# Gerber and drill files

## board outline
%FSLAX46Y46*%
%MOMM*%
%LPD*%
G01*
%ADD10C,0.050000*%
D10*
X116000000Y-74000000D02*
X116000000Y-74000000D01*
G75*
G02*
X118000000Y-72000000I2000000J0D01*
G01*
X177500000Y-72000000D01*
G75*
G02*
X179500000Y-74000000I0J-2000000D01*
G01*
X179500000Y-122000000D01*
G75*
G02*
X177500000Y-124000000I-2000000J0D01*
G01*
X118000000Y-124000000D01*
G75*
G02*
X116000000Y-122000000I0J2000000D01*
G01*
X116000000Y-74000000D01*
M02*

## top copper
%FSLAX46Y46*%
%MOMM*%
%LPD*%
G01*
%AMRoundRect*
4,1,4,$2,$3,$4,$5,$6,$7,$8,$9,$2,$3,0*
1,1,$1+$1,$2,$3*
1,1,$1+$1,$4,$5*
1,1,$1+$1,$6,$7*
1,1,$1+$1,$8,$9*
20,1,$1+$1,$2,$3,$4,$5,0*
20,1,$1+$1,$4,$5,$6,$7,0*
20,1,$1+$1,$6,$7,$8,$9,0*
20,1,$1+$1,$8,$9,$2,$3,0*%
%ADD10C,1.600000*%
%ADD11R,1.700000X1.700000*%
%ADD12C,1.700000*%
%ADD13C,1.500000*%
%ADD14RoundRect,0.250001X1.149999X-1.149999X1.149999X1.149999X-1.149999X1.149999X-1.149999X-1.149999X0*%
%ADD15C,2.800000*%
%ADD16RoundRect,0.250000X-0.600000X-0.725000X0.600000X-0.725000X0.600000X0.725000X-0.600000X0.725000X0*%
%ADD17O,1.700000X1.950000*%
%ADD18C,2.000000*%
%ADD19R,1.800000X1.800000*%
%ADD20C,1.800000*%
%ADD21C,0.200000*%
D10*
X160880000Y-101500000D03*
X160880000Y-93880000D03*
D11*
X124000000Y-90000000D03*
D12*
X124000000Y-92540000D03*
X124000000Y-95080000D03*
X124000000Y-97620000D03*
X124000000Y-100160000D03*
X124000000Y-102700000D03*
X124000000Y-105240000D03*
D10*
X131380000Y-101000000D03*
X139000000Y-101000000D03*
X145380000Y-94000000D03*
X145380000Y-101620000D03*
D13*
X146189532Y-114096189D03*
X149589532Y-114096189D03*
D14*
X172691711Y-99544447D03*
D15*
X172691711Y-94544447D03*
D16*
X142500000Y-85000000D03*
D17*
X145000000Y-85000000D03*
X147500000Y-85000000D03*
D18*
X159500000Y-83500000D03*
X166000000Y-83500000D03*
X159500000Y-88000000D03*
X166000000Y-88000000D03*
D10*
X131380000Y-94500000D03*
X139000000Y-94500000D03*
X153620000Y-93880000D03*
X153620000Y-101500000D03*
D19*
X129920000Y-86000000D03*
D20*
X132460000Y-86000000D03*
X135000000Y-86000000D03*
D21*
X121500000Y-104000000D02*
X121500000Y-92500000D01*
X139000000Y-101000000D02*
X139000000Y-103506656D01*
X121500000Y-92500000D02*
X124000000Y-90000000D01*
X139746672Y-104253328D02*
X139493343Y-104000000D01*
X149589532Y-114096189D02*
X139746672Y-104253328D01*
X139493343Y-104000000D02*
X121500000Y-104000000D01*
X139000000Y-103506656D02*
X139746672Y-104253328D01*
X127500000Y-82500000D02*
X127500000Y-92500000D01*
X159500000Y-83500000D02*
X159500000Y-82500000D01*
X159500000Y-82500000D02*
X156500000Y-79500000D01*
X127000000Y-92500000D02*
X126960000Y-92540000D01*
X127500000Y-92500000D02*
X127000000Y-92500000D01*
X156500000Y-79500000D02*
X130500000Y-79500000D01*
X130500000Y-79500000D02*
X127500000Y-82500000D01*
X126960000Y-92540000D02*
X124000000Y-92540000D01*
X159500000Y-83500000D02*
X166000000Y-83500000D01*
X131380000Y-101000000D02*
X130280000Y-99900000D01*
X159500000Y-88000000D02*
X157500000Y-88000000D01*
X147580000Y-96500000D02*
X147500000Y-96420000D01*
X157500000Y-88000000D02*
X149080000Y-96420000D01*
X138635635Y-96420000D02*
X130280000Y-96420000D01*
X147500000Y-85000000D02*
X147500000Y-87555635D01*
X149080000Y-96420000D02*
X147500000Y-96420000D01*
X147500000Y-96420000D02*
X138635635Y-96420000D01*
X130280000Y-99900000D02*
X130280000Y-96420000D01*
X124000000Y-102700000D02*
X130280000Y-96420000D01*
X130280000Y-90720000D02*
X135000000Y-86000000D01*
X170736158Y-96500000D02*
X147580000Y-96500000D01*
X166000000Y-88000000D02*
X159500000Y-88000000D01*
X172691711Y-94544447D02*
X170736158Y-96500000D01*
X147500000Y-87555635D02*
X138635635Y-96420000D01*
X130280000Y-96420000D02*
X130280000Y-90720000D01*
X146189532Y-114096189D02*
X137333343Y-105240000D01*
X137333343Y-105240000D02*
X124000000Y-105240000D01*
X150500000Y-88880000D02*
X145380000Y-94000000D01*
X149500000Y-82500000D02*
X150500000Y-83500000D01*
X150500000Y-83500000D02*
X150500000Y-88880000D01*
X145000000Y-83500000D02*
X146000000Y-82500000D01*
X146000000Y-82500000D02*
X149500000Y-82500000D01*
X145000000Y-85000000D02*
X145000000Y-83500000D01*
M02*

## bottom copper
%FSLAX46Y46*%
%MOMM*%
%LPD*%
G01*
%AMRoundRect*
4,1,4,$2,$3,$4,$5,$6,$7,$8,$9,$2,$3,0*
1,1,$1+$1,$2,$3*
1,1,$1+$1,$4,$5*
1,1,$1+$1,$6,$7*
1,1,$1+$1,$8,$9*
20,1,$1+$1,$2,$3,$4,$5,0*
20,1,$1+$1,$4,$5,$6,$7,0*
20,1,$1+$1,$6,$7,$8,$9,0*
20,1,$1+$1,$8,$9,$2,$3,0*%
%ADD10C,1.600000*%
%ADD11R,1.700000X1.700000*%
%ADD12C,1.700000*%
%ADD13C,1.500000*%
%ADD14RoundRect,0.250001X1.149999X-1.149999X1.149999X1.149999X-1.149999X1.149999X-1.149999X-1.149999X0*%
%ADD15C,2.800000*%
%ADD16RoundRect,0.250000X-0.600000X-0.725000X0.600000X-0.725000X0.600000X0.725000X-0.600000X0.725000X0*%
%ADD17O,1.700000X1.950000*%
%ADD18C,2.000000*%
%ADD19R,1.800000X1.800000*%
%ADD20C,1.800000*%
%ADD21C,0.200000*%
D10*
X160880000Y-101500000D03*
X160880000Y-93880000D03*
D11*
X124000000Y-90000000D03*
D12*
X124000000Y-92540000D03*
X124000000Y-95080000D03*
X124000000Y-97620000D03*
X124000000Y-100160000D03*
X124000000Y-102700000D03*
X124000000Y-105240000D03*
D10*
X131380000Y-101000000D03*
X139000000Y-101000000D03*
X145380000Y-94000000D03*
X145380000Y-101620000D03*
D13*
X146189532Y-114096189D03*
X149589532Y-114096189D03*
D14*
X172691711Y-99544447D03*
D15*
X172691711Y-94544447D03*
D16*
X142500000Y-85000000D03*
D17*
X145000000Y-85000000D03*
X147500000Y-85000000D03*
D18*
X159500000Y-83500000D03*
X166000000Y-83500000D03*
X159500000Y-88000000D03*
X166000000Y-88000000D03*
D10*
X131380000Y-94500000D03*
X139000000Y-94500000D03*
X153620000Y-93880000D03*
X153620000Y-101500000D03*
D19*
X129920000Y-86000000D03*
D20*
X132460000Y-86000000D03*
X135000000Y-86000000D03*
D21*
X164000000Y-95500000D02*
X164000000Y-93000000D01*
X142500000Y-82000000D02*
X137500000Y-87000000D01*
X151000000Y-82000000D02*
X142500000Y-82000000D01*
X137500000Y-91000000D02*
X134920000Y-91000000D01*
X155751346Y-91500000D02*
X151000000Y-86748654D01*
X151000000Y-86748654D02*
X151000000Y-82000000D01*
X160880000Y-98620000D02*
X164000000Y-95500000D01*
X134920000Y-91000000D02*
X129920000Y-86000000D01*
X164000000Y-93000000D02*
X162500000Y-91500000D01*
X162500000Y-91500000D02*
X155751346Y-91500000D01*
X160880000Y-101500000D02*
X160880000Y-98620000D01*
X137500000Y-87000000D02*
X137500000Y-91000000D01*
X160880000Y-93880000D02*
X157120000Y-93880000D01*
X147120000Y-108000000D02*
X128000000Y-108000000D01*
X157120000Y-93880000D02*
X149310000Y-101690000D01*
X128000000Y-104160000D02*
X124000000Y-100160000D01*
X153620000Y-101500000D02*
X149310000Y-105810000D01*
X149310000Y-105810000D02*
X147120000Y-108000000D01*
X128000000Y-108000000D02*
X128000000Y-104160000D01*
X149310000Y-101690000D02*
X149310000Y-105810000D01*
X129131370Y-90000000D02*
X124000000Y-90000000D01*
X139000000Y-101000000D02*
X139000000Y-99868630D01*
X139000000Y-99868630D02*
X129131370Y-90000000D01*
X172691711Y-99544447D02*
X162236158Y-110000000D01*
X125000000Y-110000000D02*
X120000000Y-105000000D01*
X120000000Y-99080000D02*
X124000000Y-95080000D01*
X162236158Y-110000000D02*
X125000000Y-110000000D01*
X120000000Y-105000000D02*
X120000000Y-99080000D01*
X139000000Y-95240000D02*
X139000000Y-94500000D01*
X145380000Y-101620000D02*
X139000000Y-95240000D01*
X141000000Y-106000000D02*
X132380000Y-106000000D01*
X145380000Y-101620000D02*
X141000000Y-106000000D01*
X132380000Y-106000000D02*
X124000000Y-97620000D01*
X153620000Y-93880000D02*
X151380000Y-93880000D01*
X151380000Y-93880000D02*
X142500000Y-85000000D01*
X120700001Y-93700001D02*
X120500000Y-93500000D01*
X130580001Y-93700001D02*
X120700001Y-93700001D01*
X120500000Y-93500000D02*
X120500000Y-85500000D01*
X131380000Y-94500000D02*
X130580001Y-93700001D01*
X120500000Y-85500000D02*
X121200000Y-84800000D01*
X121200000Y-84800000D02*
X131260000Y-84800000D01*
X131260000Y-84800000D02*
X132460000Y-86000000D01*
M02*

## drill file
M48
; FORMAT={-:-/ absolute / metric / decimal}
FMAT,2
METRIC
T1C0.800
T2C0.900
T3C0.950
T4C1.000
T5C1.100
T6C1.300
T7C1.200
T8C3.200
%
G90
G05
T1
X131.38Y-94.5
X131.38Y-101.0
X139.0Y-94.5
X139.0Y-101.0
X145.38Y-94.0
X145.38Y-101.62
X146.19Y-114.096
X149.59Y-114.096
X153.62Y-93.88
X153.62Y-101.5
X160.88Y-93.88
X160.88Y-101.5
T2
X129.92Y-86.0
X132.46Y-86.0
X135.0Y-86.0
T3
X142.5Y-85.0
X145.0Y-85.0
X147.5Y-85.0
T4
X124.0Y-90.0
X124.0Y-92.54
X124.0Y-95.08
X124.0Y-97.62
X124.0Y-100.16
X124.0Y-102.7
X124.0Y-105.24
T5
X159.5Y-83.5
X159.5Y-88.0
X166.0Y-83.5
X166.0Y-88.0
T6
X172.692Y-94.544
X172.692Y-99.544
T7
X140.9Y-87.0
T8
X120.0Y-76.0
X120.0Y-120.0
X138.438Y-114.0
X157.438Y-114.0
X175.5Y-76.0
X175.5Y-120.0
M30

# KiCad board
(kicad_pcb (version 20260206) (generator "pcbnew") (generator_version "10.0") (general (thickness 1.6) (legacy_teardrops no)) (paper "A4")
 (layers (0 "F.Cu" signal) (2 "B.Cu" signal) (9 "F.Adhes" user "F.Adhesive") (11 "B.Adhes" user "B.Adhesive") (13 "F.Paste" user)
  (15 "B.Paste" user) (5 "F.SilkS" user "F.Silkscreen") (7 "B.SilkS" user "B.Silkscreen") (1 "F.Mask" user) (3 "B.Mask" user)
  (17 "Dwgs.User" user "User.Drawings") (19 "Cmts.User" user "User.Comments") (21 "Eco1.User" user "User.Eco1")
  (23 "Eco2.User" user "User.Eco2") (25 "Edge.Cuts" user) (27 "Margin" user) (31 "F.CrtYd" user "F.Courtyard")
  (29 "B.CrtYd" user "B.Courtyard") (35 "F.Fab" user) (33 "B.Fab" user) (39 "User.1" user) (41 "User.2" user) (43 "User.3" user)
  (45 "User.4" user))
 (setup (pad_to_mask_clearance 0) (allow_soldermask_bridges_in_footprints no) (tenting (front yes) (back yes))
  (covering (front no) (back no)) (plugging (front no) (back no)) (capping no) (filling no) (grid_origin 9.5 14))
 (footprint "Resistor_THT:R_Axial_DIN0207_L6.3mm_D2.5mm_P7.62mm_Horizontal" (layer "F.Cu") (at 160.88 101.5 90)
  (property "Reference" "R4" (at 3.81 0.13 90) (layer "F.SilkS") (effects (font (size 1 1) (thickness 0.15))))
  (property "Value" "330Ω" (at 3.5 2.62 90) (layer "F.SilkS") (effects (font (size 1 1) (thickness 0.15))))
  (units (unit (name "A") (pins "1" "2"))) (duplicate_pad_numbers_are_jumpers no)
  (pad "1" thru_hole circle (at 0 0 90) (size 1.6 1.6) (drill 0.8) (layers "*.Cu" "*.Mask") (remove_unused_layers no) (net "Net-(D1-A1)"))
  (pad "2" thru_hole circle (at 7.62 0 90) (size 1.6 1.6) (drill 0.8) (layers "*.Cu" "*.Mask") (remove_unused_layers no) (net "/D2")))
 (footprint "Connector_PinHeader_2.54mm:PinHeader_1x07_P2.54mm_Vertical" (layer "F.Cu") (at 124 90)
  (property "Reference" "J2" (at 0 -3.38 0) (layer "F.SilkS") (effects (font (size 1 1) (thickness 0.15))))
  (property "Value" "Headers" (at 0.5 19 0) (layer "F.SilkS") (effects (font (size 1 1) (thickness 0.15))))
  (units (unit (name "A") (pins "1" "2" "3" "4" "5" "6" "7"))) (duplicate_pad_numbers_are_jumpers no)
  (pad "1" thru_hole rect (at 0 0) (size 1.7 1.7) (drill 1) (layers "*.Cu" "*.Mask") (remove_unused_layers no) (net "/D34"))
  (pad "2" thru_hole circle (at 0 2.54) (size 1.7 1.7) (drill 1) (layers "*.Cu" "*.Mask") (remove_unused_layers no) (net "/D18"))
  (pad "3" thru_hole circle (at 0 5.08) (size 1.7 1.7) (drill 1) (layers "*.Cu" "*.Mask") (remove_unused_layers no) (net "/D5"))
  (pad "4" thru_hole circle (at 0 7.62) (size 1.7 1.7) (drill 1) (layers "*.Cu" "*.Mask") (remove_unused_layers no) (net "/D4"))
  (pad "5" thru_hole circle (at 0 10.16) (size 1.7 1.7) (drill 1) (layers "*.Cu" "*.Mask") (remove_unused_layers no) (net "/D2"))
  (pad "6" thru_hole circle (at 0 12.7) (size 1.7 1.7) (drill 1) (layers "*.Cu" "*.Mask") (remove_unused_layers no) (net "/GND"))
  (pad "7" thru_hole circle (at 0 15.24) (size 1.7 1.7) (drill 1) (layers "*.Cu" "*.Mask") (remove_unused_layers no) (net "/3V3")))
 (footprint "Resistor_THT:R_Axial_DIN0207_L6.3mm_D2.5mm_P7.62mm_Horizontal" (layer "F.Cu") (at 131.38 101)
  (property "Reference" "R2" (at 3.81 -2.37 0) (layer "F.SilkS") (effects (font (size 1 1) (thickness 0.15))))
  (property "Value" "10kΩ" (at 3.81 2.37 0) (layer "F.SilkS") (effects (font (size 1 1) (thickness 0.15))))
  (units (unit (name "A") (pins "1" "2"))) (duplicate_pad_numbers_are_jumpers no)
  (pad "1" thru_hole circle (at 0 0) (size 1.6 1.6) (drill 0.8) (layers "*.Cu" "*.Mask") (remove_unused_layers no) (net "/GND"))
  (pad "2" thru_hole circle (at 7.62 0) (size 1.6 1.6) (drill 0.8) (layers "*.Cu" "*.Mask") (remove_unused_layers no) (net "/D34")))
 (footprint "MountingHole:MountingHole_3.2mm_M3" (layer "F.Cu") (at 175.5 120)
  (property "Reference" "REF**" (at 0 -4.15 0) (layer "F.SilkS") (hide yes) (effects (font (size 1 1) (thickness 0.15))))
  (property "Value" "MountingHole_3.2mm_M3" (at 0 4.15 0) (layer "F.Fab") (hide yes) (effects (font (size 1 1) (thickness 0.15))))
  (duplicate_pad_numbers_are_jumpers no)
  (pad "" np_thru_hole circle (at 0 0) (size 3.2 3.2) (drill 3.2) (layers "*.Cu" "*.Mask")))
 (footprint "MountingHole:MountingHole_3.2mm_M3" (layer "F.Cu") (at 175.5 76)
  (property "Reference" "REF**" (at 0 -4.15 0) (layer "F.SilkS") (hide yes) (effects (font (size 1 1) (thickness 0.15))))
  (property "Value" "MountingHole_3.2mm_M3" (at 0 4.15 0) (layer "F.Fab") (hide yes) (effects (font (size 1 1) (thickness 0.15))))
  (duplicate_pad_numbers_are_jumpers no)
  (pad "" np_thru_hole circle (at 0 0) (size 3.2 3.2) (drill 3.2) (layers "*.Cu" "*.Mask")))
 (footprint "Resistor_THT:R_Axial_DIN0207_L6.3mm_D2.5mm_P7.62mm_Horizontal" (layer "F.Cu") (at 145.38 94 -90)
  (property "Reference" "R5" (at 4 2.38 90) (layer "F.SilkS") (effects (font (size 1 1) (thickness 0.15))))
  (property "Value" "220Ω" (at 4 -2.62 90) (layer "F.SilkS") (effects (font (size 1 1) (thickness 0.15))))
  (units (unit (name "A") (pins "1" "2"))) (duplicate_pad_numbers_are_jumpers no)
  (pad "1" thru_hole circle (at 0 0 270) (size 1.6 1.6) (drill 0.8) (layers "*.Cu" "*.Mask") (remove_unused_layers no)
   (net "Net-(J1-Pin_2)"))
  (pad "2" thru_hole circle (at 7.62 0 270) (size 1.6 1.6) (drill 0.8) (layers "*.Cu" "*.Mask") (remove_unused_layers no) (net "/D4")))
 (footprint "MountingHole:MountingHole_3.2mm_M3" (layer "F.Cu") (at 157.437676 114)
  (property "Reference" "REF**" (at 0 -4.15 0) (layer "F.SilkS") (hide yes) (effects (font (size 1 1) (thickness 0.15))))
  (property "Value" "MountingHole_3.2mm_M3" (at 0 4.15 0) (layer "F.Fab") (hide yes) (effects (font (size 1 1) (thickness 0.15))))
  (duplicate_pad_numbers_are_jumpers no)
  (pad "" np_thru_hole circle (at 0 0) (size 3.2 3.2) (drill 3.2) (layers "*.Cu" "*.Mask")))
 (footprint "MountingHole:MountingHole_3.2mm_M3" (layer "F.Cu") (at 120 76)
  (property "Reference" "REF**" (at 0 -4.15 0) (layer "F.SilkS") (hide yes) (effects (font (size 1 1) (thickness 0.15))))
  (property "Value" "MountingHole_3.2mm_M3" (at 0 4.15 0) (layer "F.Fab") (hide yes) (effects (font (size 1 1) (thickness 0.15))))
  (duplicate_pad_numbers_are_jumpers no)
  (pad "" np_thru_hole circle (at 0 0) (size 3.2 3.2) (drill 3.2) (layers "*.Cu" "*.Mask")))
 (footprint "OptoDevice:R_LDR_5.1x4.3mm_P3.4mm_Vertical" (layer "F.Cu") (at 146.189532 114.096189)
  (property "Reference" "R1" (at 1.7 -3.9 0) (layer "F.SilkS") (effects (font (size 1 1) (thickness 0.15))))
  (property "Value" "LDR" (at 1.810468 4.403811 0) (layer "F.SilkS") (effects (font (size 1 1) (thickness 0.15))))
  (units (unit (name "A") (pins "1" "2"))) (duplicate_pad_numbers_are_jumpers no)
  (pad "1" thru_hole circle (at 0 0) (size 1.5 1.5) (drill 0.8) (layers "*.Cu" "*.Mask") (remove_unused_layers no) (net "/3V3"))
  (pad "2" thru_hole circle (at 3.4 0) (size 1.5 1.5) (drill 0.8) (layers "*.Cu" "*.Mask") (remove_unused_layers no) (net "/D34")))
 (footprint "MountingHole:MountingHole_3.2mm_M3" (layer "F.Cu") (at 120 120)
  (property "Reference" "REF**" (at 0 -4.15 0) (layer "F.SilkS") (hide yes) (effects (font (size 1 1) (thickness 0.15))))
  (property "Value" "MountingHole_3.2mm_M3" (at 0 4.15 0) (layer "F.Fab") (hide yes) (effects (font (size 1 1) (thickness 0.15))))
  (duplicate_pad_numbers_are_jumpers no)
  (pad "" np_thru_hole circle (at 0 0) (size 3.2 3.2) (drill 3.2) (layers "*.Cu" "*.Mask")))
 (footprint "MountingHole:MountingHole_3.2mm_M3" (layer "F.Cu") (at 138.437676 114)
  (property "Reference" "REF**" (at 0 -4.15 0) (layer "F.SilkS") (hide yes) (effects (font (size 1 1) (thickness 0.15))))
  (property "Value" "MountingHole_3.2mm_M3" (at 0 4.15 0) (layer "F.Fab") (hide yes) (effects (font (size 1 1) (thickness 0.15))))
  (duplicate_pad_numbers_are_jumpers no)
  (pad "" np_thru_hole circle (at 0 0) (size 3.2 3.2) (drill 3.2) (layers "*.Cu" "*.Mask")))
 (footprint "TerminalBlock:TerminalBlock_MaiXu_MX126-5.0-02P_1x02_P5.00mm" (layer "F.Cu") (at 172.691711 99.544447 90)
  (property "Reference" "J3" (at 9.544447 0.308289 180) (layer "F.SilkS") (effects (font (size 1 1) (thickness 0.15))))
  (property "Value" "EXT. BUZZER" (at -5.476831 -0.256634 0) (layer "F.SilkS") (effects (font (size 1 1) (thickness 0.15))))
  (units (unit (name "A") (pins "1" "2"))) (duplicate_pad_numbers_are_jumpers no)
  (pad "1" thru_hole roundrect (at 0 0 90) (size 2.8 2.8) (drill 1.3) (layers "*.Cu" "*.Mask") (remove_unused_layers no)
   (roundrect_rratio 0.089286) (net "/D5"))
  (pad "2" thru_hole circle (at 5 0 90) (size 2.8 2.8) (drill 1.3) (layers "*.Cu" "*.Mask") (remove_unused_layers no) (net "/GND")))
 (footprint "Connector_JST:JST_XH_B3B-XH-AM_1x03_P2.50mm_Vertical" (layer "F.Cu") (at 142.5 85)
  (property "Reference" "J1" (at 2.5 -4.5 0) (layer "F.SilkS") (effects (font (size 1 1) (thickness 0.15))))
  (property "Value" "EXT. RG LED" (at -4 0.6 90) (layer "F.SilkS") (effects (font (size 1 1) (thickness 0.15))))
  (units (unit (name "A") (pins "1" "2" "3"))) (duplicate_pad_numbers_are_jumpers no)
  (pad "" np_thru_hole circle (at -1.6 2) (size 1.2 1.2) (drill 1.2) (layers "*.Cu" "*.Mask"))
  (pad "1" thru_hole roundrect (at 0 0) (size 1.7 1.95) (drill 0.95) (layers "*.Cu" "*.Mask") (remove_unused_layers no)
   (roundrect_rratio 0.147059) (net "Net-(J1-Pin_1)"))
  (pad "2" thru_hole oval (at 2.5 0) (size 1.7 1.95) (drill 0.95) (layers "*.Cu" "*.Mask") (remove_unused_layers no) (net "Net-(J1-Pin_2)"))
  (pad "3" thru_hole oval (at 5 0) (size 1.7 1.95) (drill 0.95) (layers "*.Cu" "*.Mask") (remove_unused_layers no) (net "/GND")))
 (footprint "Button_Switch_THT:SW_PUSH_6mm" (layer "F.Cu") (at 159.5 83.5)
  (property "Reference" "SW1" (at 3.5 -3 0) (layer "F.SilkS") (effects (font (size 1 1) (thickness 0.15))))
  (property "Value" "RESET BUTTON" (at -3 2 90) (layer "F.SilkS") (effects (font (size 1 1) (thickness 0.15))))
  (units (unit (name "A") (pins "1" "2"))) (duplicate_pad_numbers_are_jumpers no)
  (pad "1" thru_hole circle (at 0 0 90) (size 2 2) (drill 1.1) (layers "*.Cu" "*.Mask") (remove_unused_layers no) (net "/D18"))
  (pad "1" thru_hole circle (at 6.5 0 90) (size 2 2) (drill 1.1) (layers "*.Cu" "*.Mask") (remove_unused_layers no) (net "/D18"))
  (pad "2" thru_hole circle (at 0 4.5 90) (size 2 2) (drill 1.1) (layers "*.Cu" "*.Mask") (remove_unused_layers no) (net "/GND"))
  (pad "2" thru_hole circle (at 6.5 4.5 90) (size 2 2) (drill 1.1) (layers "*.Cu" "*.Mask") (remove_unused_layers no) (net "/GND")))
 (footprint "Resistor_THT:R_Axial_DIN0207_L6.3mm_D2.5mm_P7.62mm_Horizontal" (layer "F.Cu") (at 131.38 94.5)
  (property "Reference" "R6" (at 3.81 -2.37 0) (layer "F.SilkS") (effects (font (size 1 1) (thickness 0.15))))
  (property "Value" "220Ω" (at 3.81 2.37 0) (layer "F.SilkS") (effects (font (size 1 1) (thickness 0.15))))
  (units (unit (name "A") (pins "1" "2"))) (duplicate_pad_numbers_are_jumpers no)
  (pad "1" thru_hole circle (at 0 0) (size 1.6 1.6) (drill 0.8) (layers "*.Cu" "*.Mask") (remove_unused_layers no) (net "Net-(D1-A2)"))
  (pad "2" thru_hole circle (at 7.62 0) (size 1.6 1.6) (drill 0.8) (layers "*.Cu" "*.Mask") (remove_unused_layers no) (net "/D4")))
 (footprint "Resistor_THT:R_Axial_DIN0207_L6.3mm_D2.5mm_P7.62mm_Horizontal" (layer "F.Cu") (at 153.62 93.88 -90)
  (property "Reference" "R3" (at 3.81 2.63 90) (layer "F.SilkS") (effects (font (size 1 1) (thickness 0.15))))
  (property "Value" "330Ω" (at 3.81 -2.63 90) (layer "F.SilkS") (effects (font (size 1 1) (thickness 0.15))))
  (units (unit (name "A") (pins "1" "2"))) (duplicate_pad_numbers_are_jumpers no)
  (pad "1" thru_hole circle (at 0 0 270) (size 1.6 1.6) (drill 0.8) (layers "*.Cu" "*.Mask") (remove_unused_layers no)
   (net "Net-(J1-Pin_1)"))
  (pad "2" thru_hole circle (at 7.62 0 270) (size 1.6 1.6) (drill 0.8) (layers "*.Cu" "*.Mask") (remove_unused_layers no) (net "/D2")))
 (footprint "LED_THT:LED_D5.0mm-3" (layer "F.Cu") (at 129.92 86)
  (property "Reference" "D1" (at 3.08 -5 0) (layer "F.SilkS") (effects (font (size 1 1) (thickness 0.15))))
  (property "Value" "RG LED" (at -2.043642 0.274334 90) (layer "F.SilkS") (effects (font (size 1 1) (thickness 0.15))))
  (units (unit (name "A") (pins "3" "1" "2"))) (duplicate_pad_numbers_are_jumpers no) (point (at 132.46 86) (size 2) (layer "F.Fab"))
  (pad "1" thru_hole rect (at 0 0) (size 1.8 1.8) (drill 0.9) (layers "*.Cu" "*.Mask") (remove_unused_layers no) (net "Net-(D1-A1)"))
  (pad "2" thru_hole circle (at 2.54 0) (size 1.8 1.8) (drill 0.9) (layers "*.Cu" "*.Mask") (remove_unused_layers no) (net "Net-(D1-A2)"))
  (pad "3" thru_hole circle (at 5.08 0) (size 1.8 1.8) (drill 0.9) (layers "*.Cu" "*.Mask") (remove_unused_layers no) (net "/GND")))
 (gr_rect (start 116 72) (end 179.5 124) (radius 2) (stroke (width 0.05) (type default)) (fill no) (layer "Edge.Cuts"))
 (segment (start 164 95.5) (end 164 93) (width 0.2) (layer "B.Cu") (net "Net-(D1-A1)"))
 (segment (start 142.5 82) (end 137.5 87) (width 0.2) (layer "B.Cu") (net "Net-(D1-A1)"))
 (segment (start 151 82) (end 142.5 82) (width 0.2) (layer "B.Cu") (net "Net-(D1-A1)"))
 (segment (start 137.5 91) (end 134.92 91) (width 0.2) (layer "B.Cu") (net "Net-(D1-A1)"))
 (segment (start 155.751346 91.5) (end 151 86.748654) (width 0.2) (layer "B.Cu") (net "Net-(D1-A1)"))
 (segment (start 151 86.748654) (end 151 82) (width 0.2) (layer "B.Cu") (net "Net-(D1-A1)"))
 (segment (start 160.88 98.62) (end 164 95.5) (width 0.2) (layer "B.Cu") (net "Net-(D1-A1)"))
 (segment (start 134.92 91) (end 129.92 86) (width 0.2) (layer "B.Cu") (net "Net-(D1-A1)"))
 (segment (start 164 93) (end 162.5 91.5) (width 0.2) (layer "B.Cu") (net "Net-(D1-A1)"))
 (segment (start 162.5 91.5) (end 155.751346 91.5) (width 0.2) (layer "B.Cu") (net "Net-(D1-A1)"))
 (segment (start 160.88 101.5) (end 160.88 98.62) (width 0.2) (layer "B.Cu") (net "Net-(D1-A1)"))
 (segment (start 137.5 87) (end 137.5 91) (width 0.2) (layer "B.Cu") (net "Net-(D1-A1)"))
 (segment (start 160.88 93.88) (end 157.12 93.88) (width 0.2) (layer "B.Cu") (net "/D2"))
 (segment (start 147.12 108) (end 128 108) (width 0.2) (layer "B.Cu") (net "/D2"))
 (segment (start 157.12 93.88) (end 149.31 101.69) (width 0.2) (layer "B.Cu") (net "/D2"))
 (segment (start 128 104.16) (end 124 100.16) (width 0.2) (layer "B.Cu") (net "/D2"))
 (segment (start 153.62 101.5) (end 149.31 105.81) (width 0.2) (layer "B.Cu") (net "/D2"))
 (segment (start 149.31 105.81) (end 147.12 108) (width 0.2) (layer "B.Cu") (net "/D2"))
 (segment (start 128 108) (end 128 104.16) (width 0.2) (layer "B.Cu") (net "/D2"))
 (segment (start 149.31 101.69) (end 149.31 105.81) (width 0.2) (layer "B.Cu") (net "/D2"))
 (segment (start 121.5 104) (end 121.5 92.5) (width 0.2) (layer "F.Cu") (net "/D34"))
 (segment (start 139 101) (end 139 103.506656) (width 0.2) (layer "F.Cu") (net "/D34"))
 (segment (start 121.5 92.5) (end 124 90) (width 0.2) (layer "F.Cu") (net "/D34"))
 (segment (start 139.746672 104.253328) (end 139.493343 104) (width 0.2) (layer "F.Cu") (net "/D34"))
 (segment (start 149.589532 114.096189) (end 139.746672 104.253328) (width 0.2) (layer "F.Cu") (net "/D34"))
 (segment (start 139.493343 104) (end 121.5 104) (width 0.2) (layer "F.Cu") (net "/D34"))
 (segment (start 139 103.506656) (end 139.746672 104.253328) (width 0.2) (layer "F.Cu") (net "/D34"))
 (segment (start 129.13137 90) (end 124 90) (width 0.2) (layer "B.Cu") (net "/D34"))
 (segment (start 139 101) (end 139 99.86863) (width 0.2) (layer "B.Cu") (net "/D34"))
 (segment (start 139 99.86863) (end 129.13137 90) (width 0.2) (layer "B.Cu") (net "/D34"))
 (segment (start 127.5 82.5) (end 127.5 92.5) (width 0.2) (layer "F.Cu") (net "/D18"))
 (segment (start 159.5 83.5) (end 159.5 82.5) (width 0.2) (layer "F.Cu") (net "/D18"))
 (segment (start 159.5 82.5) (end 156.5 79.5) (width 0.2) (layer "F.Cu") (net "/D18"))
 (segment (start 127 92.5) (end 126.96 92.54) (width 0.2) (layer "F.Cu") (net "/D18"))
 (segment (start 127.5 92.5) (end 127 92.5) (width 0.2) (layer "F.Cu") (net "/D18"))
 (segment (start 156.5 79.5) (end 130.5 79.5) (width 0.2) (layer "F.Cu") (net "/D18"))
 (segment (start 130.5 79.5) (end 127.5 82.5) (width 0.2) (layer "F.Cu") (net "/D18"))
 (segment (start 126.96 92.54) (end 124 92.54) (width 0.2) (layer "F.Cu") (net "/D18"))
 (segment (start 159.5 83.5) (end 166 83.5) (width 0.2) (layer "F.Cu") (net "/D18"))
 (segment (start 172.691711 99.544447) (end 162.236158 110) (width 0.2) (layer "B.Cu") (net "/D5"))
 (segment (start 125 110) (end 120 105) (width 0.2) (layer "B.Cu") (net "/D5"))
 (segment (start 120 99.08) (end 124 95.08) (width 0.2) (layer "B.Cu") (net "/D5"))
 (segment (start 162.236158 110) (end 125 110) (width 0.2) (layer "B.Cu") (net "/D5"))
 (segment (start 120 105) (end 120 99.08) (width 0.2) (layer "B.Cu") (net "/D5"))
 (segment (start 139 95.24) (end 139 94.5) (width 0.2) (layer "B.Cu") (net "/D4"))
 (segment (start 145.38 101.62) (end 139 95.24) (width 0.2) (layer "B.Cu") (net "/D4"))
 (segment (start 141 106) (end 132.38 106) (width 0.2) (layer "B.Cu") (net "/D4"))
 (segment (start 145.38 101.62) (end 141 106) (width 0.2) (layer "B.Cu") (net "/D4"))
 (segment (start 132.38 106) (end 124 97.62) (width 0.2) (layer "B.Cu") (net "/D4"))
 (segment (start 131.38 101) (end 130.28 99.9) (width 0.2) (layer "F.Cu") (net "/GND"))
 (segment (start 159.5 88) (end 157.5 88) (width 0.2) (layer "F.Cu") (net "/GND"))
 (segment (start 147.58 96.5) (end 147.5 96.42) (width 0.2) (layer "F.Cu") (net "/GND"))
 (segment (start 157.5 88) (end 149.08 96.42) (width 0.2) (layer "F.Cu") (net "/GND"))
 (segment (start 138.635635 96.42) (end 130.28 96.42) (width 0.2) (layer "F.Cu") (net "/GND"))
 (segment (start 147.5 85) (end 147.5 87.555635) (width 0.2) (layer "F.Cu") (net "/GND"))
 (segment (start 149.08 96.42) (end 147.5 96.42) (width 0.2) (layer "F.Cu") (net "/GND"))
 (segment (start 147.5 96.42) (end 138.635635 96.42) (width 0.2) (layer "F.Cu") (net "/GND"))
 (segment (start 130.28 99.9) (end 130.28 96.42) (width 0.2) (layer "F.Cu") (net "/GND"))
 (segment (start 124 102.7) (end 130.28 96.42) (width 0.2) (layer "F.Cu") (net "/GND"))
 (segment (start 130.28 90.72) (end 135 86) (width 0.2) (layer "F.Cu") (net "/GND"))
 (segment (start 170.736158 96.5) (end 147.58 96.5) (width 0.2) (layer "F.Cu") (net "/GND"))
 (segment (start 166 88) (end 159.5 88) (width 0.2) (layer "F.Cu") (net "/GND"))
 (segment (start 172.691711 94.544447) (end 170.736158 96.5) (width 0.2) (layer "F.Cu") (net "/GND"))
 (segment (start 147.5 87.555635) (end 138.635635 96.42) (width 0.2) (layer "F.Cu") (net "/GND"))
 (segment (start 130.28 96.42) (end 130.28 90.72) (width 0.2) (layer "F.Cu") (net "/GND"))
 (segment (start 146.189532 114.096189) (end 137.333343 105.24) (width 0.2) (layer "F.Cu") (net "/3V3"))
 (segment (start 137.333343 105.24) (end 124 105.24) (width 0.2) (layer "F.Cu") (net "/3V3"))
 (segment (start 150.5 88.88) (end 145.38 94) (width 0.2) (layer "F.Cu") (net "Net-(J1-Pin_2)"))
 (segment (start 149.5 82.5) (end 150.5 83.5) (width 0.2) (layer "F.Cu") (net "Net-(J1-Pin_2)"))
 (segment (start 150.5 83.5) (end 150.5 88.88) (width 0.2) (layer "F.Cu") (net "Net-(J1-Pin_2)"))
 (segment (start 145 83.5) (end 146 82.5) (width 0.2) (layer "F.Cu") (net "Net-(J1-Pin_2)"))
 (segment (start 146 82.5) (end 149.5 82.5) (width 0.2) (layer "F.Cu") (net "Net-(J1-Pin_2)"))
 (segment (start 145 85) (end 145 83.5) (width 0.2) (layer "F.Cu") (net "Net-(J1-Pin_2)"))
 (segment (start 153.62 93.88) (end 151.38 93.88) (width 0.2) (layer "B.Cu") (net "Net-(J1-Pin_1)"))
 (segment (start 151.38 93.88) (end 142.5 85) (width 0.2) (layer "B.Cu") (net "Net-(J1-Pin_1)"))
 (segment (start 120.700001 93.700001) (end 120.5 93.5) (width 0.2) (layer "B.Cu") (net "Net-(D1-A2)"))
 (segment (start 130.580001 93.700001) (end 120.700001 93.700001) (width 0.2) (layer "B.Cu") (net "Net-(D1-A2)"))
 (segment (start 120.5 93.5) (end 120.5 85.5) (width 0.2) (layer "B.Cu") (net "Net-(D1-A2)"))
 (segment (start 131.38 94.5) (end 130.580001 93.700001) (width 0.2) (layer "B.Cu") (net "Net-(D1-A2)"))
 (segment (start 120.5 85.5) (end 121.2 84.8) (width 0.2) (layer "B.Cu") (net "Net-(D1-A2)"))
 (segment (start 121.2 84.8) (end 131.26 84.8) (width 0.2) (layer "B.Cu") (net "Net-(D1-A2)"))
 (segment (start 131.26 84.8) (end 132.46 86) (width 0.2) (layer "B.Cu") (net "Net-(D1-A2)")))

